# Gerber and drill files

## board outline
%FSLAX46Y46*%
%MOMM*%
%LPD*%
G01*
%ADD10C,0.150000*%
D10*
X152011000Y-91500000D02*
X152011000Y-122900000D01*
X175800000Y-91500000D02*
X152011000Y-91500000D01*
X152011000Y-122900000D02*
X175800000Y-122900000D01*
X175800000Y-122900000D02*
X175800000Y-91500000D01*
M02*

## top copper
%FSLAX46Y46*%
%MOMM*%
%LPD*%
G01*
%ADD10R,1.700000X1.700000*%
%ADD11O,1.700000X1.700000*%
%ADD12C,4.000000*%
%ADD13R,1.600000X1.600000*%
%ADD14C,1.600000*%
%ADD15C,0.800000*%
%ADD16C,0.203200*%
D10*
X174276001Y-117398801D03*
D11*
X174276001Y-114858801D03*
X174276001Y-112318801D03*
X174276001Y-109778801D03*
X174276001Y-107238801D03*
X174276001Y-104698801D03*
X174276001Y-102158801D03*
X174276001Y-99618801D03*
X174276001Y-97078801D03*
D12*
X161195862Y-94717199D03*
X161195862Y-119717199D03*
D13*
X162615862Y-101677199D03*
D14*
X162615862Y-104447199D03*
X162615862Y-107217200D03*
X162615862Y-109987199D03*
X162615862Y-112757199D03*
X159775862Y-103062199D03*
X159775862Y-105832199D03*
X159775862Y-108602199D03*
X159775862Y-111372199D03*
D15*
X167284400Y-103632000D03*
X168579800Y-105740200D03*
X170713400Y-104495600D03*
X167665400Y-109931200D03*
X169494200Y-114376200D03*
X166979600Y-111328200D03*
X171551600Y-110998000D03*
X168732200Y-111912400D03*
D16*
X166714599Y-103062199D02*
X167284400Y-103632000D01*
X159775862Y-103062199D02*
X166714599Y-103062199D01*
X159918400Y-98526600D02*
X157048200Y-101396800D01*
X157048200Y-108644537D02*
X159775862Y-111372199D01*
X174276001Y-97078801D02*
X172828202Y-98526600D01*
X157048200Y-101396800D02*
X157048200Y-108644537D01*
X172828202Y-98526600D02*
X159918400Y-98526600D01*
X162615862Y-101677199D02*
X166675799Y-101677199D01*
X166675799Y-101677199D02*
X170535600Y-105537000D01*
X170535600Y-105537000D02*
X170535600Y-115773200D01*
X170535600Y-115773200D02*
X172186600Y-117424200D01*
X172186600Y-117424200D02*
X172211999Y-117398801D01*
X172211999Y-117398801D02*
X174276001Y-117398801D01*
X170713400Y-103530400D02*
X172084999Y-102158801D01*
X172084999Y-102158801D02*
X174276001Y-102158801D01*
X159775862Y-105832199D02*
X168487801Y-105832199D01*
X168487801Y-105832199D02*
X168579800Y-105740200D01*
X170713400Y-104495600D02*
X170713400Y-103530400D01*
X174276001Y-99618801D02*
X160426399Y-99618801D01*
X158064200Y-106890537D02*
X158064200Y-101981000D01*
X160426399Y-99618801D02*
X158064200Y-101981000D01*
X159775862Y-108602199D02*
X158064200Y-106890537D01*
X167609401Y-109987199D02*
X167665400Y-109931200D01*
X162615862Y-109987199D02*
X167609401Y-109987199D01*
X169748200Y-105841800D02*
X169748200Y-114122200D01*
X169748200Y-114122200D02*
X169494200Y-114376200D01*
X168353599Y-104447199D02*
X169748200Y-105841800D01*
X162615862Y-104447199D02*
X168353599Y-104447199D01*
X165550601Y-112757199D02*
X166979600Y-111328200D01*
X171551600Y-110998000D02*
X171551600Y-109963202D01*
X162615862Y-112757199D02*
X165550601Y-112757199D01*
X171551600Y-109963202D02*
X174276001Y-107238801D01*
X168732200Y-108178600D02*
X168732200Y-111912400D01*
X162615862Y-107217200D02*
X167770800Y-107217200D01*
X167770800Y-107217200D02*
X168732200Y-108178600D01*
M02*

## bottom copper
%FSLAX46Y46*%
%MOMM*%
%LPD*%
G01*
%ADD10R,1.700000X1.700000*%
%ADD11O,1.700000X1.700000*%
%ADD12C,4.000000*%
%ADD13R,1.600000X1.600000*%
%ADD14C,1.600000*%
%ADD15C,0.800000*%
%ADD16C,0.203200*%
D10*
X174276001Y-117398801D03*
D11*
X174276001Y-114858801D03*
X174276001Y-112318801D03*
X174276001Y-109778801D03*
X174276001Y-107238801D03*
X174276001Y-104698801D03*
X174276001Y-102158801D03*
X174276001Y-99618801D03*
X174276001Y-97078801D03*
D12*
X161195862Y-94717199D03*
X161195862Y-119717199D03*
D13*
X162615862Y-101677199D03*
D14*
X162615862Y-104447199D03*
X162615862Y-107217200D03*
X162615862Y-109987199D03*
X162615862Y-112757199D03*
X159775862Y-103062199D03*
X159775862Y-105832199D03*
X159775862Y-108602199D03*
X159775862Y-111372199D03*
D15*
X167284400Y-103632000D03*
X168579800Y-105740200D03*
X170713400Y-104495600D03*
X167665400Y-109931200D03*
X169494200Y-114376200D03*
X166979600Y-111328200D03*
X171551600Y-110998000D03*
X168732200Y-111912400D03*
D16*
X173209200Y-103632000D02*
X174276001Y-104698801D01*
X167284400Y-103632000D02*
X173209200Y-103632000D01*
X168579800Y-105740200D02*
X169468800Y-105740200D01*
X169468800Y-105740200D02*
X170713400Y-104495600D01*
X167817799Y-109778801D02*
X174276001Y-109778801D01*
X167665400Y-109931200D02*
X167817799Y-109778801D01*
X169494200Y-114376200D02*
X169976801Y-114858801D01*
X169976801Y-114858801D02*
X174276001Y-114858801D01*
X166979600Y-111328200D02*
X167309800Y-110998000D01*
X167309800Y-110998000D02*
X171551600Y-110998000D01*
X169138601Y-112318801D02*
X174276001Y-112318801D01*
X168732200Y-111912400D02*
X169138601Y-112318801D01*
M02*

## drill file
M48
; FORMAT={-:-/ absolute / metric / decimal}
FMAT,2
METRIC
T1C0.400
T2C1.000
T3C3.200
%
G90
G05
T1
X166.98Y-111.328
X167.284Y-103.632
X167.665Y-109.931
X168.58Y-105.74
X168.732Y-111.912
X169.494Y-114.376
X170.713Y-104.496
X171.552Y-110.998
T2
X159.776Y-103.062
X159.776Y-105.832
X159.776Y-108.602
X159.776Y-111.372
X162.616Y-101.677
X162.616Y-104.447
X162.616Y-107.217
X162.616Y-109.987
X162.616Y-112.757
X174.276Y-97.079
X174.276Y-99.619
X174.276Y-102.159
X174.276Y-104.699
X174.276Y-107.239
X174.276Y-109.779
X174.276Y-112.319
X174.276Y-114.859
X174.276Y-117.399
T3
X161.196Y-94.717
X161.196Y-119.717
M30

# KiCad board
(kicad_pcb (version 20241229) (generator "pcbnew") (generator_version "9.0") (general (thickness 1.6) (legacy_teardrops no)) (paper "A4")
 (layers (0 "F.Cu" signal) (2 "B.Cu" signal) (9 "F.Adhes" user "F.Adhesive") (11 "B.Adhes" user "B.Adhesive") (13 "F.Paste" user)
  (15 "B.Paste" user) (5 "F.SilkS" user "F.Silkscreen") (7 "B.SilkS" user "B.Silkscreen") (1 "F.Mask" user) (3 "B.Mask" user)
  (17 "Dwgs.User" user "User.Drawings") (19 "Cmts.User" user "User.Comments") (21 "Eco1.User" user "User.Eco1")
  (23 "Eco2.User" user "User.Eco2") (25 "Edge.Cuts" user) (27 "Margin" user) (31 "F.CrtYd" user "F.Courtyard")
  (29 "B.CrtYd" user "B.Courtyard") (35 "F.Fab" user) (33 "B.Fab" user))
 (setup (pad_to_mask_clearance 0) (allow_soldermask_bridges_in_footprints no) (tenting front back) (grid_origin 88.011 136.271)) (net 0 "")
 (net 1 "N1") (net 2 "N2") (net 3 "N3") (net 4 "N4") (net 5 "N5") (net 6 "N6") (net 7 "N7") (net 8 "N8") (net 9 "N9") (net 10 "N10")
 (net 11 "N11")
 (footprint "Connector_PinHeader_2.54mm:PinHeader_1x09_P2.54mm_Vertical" (layer "F.Cu") (at 174.276001 117.398801 180)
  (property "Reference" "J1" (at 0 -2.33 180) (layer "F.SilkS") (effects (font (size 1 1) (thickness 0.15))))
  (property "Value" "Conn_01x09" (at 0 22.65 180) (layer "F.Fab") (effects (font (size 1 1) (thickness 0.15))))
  (pad "1" thru_hole rect (at 0 0 180) (size 1.7 1.7) (drill 1) (layers "*.Cu" "*.Mask") (remove_unused_layers no) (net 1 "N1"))
  (pad "2" thru_hole oval (at 0 2.54 180) (size 1.7 1.7) (drill 1) (layers "*.Cu" "*.Mask") (remove_unused_layers no) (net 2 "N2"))
  (pad "3" thru_hole oval (at 0 5.08 180) (size 1.7 1.7) (drill 1) (layers "*.Cu" "*.Mask") (remove_unused_layers no) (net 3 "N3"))
  (pad "4" thru_hole oval (at 0 7.62 180) (size 1.7 1.7) (drill 1) (layers "*.Cu" "*.Mask") (remove_unused_layers no) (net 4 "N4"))
  (pad "5" thru_hole oval (at 0 10.16 180) (size 1.7 1.7) (drill 1) (layers "*.Cu" "*.Mask") (remove_unused_layers no) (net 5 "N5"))
  (pad "6" thru_hole oval (at 0 12.7 180) (size 1.7 1.7) (drill 1) (layers "*.Cu" "*.Mask") (remove_unused_layers no) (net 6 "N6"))
  (pad "7" thru_hole oval (at 0 15.24 180) (size 1.7 1.7) (drill 1) (layers "*.Cu" "*.Mask") (remove_unused_layers no) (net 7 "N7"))
  (pad "8" thru_hole oval (at 0 17.78 180) (size 1.7 1.7) (drill 1) (layers "*.Cu" "*.Mask") (remove_unused_layers no) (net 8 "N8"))
  (pad "9" thru_hole oval (at 0 20.32 180) (size 1.7 1.7) (drill 1) (layers "*.Cu" "*.Mask") (remove_unused_layers no) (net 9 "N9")))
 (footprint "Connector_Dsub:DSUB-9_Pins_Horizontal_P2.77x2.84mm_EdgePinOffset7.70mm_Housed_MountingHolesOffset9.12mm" (layer "F.Cu")
  (at 162.615862 101.677199 -90)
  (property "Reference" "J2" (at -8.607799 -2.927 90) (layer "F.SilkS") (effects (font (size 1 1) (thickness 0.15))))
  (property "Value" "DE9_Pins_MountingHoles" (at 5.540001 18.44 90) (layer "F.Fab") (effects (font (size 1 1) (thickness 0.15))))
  (pad "0" thru_hole circle (at -6.96 1.42 270) (size 4 4) (drill 3.2) (layers "*.Cu" "*.Mask") (remove_unused_layers no) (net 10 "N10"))
  (pad "0" thru_hole circle (at 18.04 1.42 270) (size 4 4) (drill 3.2) (layers "*.Cu" "*.Mask") (remove_unused_layers no) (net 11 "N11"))
  (pad "1" thru_hole rect (at 0 0 270) (size 1.6 1.6) (drill 1) (layers "*.Cu" "*.Mask") (remove_unused_layers no) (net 1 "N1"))
  (pad "2" thru_hole circle (at 2.77 0 270) (size 1.6 1.6) (drill 1) (layers "*.Cu" "*.Mask") (remove_unused_layers no) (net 2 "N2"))
  (pad "3" thru_hole circle (at 5.540001 0 270) (size 1.6 1.6) (drill 1) (layers "*.Cu" "*.Mask") (remove_unused_layers no) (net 3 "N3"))
  (pad "4" thru_hole circle (at 8.31 0 270) (size 1.6 1.6) (drill 1) (layers "*.Cu" "*.Mask") (remove_unused_layers no) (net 4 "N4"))
  (pad "5" thru_hole circle (at 11.08 0 270) (size 1.6 1.6) (drill 1) (layers "*.Cu" "*.Mask") (remove_unused_layers no) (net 5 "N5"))
  (pad "6" thru_hole circle (at 1.385 2.84 270) (size 1.6 1.6) (drill 1) (layers "*.Cu" "*.Mask") (remove_unused_layers no) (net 6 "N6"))
  (pad "7" thru_hole circle (at 4.155 2.84 270) (size 1.6 1.6) (drill 1) (layers "*.Cu" "*.Mask") (remove_unused_layers no) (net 7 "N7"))
  (pad "8" thru_hole circle (at 6.925 2.84 270) (size 1.6 1.6) (drill 1) (layers "*.Cu" "*.Mask") (remove_unused_layers no) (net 8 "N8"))
  (pad "9" thru_hole circle (at 9.695 2.84 270) (size 1.6 1.6) (drill 1) (layers "*.Cu" "*.Mask") (remove_unused_layers no) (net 9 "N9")))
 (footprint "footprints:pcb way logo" (layer "B.Cu") (at 156.8196 107.6452 -90)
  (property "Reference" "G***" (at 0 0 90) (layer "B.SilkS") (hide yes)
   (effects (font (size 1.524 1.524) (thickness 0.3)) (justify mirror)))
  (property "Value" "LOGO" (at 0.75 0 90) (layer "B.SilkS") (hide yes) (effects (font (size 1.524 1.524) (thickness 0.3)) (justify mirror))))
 (gr_line (start 152.011 91.5) (end 152.011 122.9) (stroke (width 0.15) (type solid)) (layer "Edge.Cuts"))
 (gr_line (start 175.8 91.5) (end 152.011 91.5) (stroke (width 0.15) (type solid)) (layer "Edge.Cuts"))
 (gr_line (start 152.011 122.9) (end 175.8 122.9) (stroke (width 0.15) (type solid)) (layer "Edge.Cuts"))
 (gr_line (start 175.8 122.9) (end 175.8 91.5) (stroke (width 0.15) (type solid)) (layer "Edge.Cuts"))
 (segment (start 166.714599 103.062199) (end 167.2844 103.632) (width 0.2032) (layer "F.Cu") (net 6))
 (segment (start 159.775862 103.062199) (end 166.714599 103.062199) (width 0.2032) (layer "F.Cu") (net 6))
 (via (at 167.2844 103.632) (size 0.8) (drill 0.4) (layers "F.Cu" "B.Cu") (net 6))
 (segment (start 173.2092 103.632) (end 174.276001 104.698801) (width 0.2032) (layer "B.Cu") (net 6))
 (segment (start 167.2844 103.632) (end 173.2092 103.632) (width 0.2032) (layer "B.Cu") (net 6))
 (segment (start 159.9184 98.5266) (end 157.0482 101.3968) (width 0.2032) (layer "F.Cu") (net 9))
 (segment (start 157.0482 108.644537) (end 159.775862 111.372199) (width 0.2032) (layer "F.Cu") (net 9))
 (segment (start 174.276001 97.078801) (end 172.828202 98.5266) (width 0.2032) (layer "F.Cu") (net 9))
 (segment (start 157.0482 101.3968) (end 157.0482 108.644537) (width 0.2032) (layer "F.Cu") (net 9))
 (segment (start 172.828202 98.5266) (end 159.9184 98.5266) (width 0.2032) (layer "F.Cu") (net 9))
 (segment (start 162.615862 101.677199) (end 166.675799 101.677199) (width 0.2032) (layer "F.Cu") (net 1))
 (segment (start 166.675799 101.677199) (end 170.5356 105.537) (width 0.2032) (layer "F.Cu") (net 1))
 (segment (start 170.5356 105.537) (end 170.5356 115.7732) (width 0.2032) (layer "F.Cu") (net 1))
 (segment (start 170.5356 115.7732) (end 172.1866 117.4242) (width 0.2032) (layer "F.Cu") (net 1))
 (segment (start 172.1866 117.4242) (end 172.211999 117.398801) (width 0.2032) (layer "F.Cu") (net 1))
 (segment (start 172.211999 117.398801) (end 174.276001 117.398801) (width 0.2032) (layer "F.Cu") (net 1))
 (segment (start 170.7134 103.5304) (end 172.084999 102.158801) (width 0.2032) (layer "F.Cu") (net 7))
 (segment (start 172.084999 102.158801) (end 174.276001 102.158801) (width 0.2032) (layer "F.Cu") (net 7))
 (segment (start 159.775862 105.832199) (end 168.487801 105.832199) (width 0.2032) (layer "F.Cu") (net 7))
 (segment (start 168.487801 105.832199) (end 168.5798 105.7402) (width 0.2032) (layer "F.Cu") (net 7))
 (segment (start 170.7134 104.4956) (end 170.7134 103.5304) (width 0.2032) (layer "F.Cu") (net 7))
 (via (at 168.5798 105.7402) (size 0.8) (drill 0.4) (layers "F.Cu" "B.Cu") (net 7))
 (via (at 170.7134 104.4956) (size 0.8) (drill 0.4) (layers "F.Cu" "B.Cu") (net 7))
 (segment (start 168.5798 105.7402) (end 169.4688 105.7402) (width 0.2032) (layer "B.Cu") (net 7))
 (segment (start 169.4688 105.7402) (end 170.7134 104.4956) (width 0.2032) (layer "B.Cu") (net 7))
 (segment (start 174.276001 99.618801) (end 160.426399 99.618801) (width 0.2032) (layer "F.Cu") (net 8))
 (segment (start 158.0642 106.890537) (end 158.0642 101.981) (width 0.2032) (layer "F.Cu") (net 8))
 (segment (start 160.426399 99.618801) (end 158.0642 101.981) (width 0.2032) (layer "F.Cu") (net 8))
 (segment (start 159.775862 108.602199) (end 158.0642 106.890537) (width 0.2032) (layer "F.Cu") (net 8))
 (segment (start 167.609401 109.987199) (end 167.6654 109.9312) (width 0.2032) (layer "F.Cu") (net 4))
 (segment (start 162.615862 109.987199) (end 167.609401 109.987199) (width 0.2032) (layer "F.Cu") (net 4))
 (via (at 167.6654 109.9312) (size 0.8) (drill 0.4) (layers "F.Cu" "B.Cu") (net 4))
 (segment (start 167.817799 109.778801) (end 174.276001 109.778801) (width 0.2032) (layer "B.Cu") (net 4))
 (segment (start 167.6654 109.9312) (end 167.817799 109.778801) (width 0.2032) (layer "B.Cu") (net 4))
 (segment (start 169.7482 105.8418) (end 169.7482 114.1222) (width 0.2032) (layer "F.Cu") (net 2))
 (segment (start 169.7482 114.1222) (end 169.4942 114.3762) (width 0.2032) (layer "F.Cu") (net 2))
 (segment (start 168.353599 104.447199) (end 169.7482 105.8418) (width 0.2032) (layer "F.Cu") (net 2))
 (segment (start 162.615862 104.447199) (end 168.353599 104.447199) (width 0.2032) (layer "F.Cu") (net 2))
 (via (at 169.4942 114.3762) (size 0.8) (drill 0.4) (layers "F.Cu" "B.Cu") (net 2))
 (segment (start 169.4942 114.3762) (end 169.976801 114.858801) (width 0.2032) (layer "B.Cu") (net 2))
 (segment (start 169.976801 114.858801) (end 174.276001 114.858801) (width 0.2032) (layer "B.Cu") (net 2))
 (segment (start 165.550601 112.757199) (end 166.9796 111.3282) (width 0.2032) (layer "F.Cu") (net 5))
 (segment (start 171.5516 110.998) (end 171.5516 109.963202) (width 0.2032) (layer "F.Cu") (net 5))
 (segment (start 162.615862 112.757199) (end 165.550601 112.757199) (width 0.2032) (layer "F.Cu") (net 5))
 (segment (start 171.5516 109.963202) (end 174.276001 107.238801) (width 0.2032) (layer "F.Cu") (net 5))
 (via (at 166.9796 111.3282) (size 0.8) (drill 0.4) (layers "F.Cu" "B.Cu") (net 5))
 (via (at 171.5516 110.998) (size 0.8) (drill 0.4) (layers "F.Cu" "B.Cu") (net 5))
 (segment (start 166.9796 111.3282) (end 167.3098 110.998) (width 0.2032) (layer "B.Cu") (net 5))
 (segment (start 167.3098 110.998) (end 171.5516 110.998) (width 0.2032) (layer "B.Cu") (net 5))
 (segment (start 168.7322 108.1786) (end 168.7322 111.9124) (width 0.2032) (layer "F.Cu") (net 3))
 (segment (start 162.615862 107.2172) (end 167.7708 107.2172) (width 0.2032) (layer "F.Cu") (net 3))
 (segment (start 167.7708 107.2172) (end 168.7322 108.1786) (width 0.2032) (layer "F.Cu") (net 3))
 (via (at 168.7322 111.9124) (size 0.8) (drill 0.4) (layers "F.Cu" "B.Cu") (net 3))
 (segment (start 169.138601 112.318801) (end 174.276001 112.318801) (width 0.2032) (layer "B.Cu") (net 3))
 (segment (start 168.7322 111.9124) (end 169.138601 112.318801) (width 0.2032) (layer "B.Cu") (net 3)))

